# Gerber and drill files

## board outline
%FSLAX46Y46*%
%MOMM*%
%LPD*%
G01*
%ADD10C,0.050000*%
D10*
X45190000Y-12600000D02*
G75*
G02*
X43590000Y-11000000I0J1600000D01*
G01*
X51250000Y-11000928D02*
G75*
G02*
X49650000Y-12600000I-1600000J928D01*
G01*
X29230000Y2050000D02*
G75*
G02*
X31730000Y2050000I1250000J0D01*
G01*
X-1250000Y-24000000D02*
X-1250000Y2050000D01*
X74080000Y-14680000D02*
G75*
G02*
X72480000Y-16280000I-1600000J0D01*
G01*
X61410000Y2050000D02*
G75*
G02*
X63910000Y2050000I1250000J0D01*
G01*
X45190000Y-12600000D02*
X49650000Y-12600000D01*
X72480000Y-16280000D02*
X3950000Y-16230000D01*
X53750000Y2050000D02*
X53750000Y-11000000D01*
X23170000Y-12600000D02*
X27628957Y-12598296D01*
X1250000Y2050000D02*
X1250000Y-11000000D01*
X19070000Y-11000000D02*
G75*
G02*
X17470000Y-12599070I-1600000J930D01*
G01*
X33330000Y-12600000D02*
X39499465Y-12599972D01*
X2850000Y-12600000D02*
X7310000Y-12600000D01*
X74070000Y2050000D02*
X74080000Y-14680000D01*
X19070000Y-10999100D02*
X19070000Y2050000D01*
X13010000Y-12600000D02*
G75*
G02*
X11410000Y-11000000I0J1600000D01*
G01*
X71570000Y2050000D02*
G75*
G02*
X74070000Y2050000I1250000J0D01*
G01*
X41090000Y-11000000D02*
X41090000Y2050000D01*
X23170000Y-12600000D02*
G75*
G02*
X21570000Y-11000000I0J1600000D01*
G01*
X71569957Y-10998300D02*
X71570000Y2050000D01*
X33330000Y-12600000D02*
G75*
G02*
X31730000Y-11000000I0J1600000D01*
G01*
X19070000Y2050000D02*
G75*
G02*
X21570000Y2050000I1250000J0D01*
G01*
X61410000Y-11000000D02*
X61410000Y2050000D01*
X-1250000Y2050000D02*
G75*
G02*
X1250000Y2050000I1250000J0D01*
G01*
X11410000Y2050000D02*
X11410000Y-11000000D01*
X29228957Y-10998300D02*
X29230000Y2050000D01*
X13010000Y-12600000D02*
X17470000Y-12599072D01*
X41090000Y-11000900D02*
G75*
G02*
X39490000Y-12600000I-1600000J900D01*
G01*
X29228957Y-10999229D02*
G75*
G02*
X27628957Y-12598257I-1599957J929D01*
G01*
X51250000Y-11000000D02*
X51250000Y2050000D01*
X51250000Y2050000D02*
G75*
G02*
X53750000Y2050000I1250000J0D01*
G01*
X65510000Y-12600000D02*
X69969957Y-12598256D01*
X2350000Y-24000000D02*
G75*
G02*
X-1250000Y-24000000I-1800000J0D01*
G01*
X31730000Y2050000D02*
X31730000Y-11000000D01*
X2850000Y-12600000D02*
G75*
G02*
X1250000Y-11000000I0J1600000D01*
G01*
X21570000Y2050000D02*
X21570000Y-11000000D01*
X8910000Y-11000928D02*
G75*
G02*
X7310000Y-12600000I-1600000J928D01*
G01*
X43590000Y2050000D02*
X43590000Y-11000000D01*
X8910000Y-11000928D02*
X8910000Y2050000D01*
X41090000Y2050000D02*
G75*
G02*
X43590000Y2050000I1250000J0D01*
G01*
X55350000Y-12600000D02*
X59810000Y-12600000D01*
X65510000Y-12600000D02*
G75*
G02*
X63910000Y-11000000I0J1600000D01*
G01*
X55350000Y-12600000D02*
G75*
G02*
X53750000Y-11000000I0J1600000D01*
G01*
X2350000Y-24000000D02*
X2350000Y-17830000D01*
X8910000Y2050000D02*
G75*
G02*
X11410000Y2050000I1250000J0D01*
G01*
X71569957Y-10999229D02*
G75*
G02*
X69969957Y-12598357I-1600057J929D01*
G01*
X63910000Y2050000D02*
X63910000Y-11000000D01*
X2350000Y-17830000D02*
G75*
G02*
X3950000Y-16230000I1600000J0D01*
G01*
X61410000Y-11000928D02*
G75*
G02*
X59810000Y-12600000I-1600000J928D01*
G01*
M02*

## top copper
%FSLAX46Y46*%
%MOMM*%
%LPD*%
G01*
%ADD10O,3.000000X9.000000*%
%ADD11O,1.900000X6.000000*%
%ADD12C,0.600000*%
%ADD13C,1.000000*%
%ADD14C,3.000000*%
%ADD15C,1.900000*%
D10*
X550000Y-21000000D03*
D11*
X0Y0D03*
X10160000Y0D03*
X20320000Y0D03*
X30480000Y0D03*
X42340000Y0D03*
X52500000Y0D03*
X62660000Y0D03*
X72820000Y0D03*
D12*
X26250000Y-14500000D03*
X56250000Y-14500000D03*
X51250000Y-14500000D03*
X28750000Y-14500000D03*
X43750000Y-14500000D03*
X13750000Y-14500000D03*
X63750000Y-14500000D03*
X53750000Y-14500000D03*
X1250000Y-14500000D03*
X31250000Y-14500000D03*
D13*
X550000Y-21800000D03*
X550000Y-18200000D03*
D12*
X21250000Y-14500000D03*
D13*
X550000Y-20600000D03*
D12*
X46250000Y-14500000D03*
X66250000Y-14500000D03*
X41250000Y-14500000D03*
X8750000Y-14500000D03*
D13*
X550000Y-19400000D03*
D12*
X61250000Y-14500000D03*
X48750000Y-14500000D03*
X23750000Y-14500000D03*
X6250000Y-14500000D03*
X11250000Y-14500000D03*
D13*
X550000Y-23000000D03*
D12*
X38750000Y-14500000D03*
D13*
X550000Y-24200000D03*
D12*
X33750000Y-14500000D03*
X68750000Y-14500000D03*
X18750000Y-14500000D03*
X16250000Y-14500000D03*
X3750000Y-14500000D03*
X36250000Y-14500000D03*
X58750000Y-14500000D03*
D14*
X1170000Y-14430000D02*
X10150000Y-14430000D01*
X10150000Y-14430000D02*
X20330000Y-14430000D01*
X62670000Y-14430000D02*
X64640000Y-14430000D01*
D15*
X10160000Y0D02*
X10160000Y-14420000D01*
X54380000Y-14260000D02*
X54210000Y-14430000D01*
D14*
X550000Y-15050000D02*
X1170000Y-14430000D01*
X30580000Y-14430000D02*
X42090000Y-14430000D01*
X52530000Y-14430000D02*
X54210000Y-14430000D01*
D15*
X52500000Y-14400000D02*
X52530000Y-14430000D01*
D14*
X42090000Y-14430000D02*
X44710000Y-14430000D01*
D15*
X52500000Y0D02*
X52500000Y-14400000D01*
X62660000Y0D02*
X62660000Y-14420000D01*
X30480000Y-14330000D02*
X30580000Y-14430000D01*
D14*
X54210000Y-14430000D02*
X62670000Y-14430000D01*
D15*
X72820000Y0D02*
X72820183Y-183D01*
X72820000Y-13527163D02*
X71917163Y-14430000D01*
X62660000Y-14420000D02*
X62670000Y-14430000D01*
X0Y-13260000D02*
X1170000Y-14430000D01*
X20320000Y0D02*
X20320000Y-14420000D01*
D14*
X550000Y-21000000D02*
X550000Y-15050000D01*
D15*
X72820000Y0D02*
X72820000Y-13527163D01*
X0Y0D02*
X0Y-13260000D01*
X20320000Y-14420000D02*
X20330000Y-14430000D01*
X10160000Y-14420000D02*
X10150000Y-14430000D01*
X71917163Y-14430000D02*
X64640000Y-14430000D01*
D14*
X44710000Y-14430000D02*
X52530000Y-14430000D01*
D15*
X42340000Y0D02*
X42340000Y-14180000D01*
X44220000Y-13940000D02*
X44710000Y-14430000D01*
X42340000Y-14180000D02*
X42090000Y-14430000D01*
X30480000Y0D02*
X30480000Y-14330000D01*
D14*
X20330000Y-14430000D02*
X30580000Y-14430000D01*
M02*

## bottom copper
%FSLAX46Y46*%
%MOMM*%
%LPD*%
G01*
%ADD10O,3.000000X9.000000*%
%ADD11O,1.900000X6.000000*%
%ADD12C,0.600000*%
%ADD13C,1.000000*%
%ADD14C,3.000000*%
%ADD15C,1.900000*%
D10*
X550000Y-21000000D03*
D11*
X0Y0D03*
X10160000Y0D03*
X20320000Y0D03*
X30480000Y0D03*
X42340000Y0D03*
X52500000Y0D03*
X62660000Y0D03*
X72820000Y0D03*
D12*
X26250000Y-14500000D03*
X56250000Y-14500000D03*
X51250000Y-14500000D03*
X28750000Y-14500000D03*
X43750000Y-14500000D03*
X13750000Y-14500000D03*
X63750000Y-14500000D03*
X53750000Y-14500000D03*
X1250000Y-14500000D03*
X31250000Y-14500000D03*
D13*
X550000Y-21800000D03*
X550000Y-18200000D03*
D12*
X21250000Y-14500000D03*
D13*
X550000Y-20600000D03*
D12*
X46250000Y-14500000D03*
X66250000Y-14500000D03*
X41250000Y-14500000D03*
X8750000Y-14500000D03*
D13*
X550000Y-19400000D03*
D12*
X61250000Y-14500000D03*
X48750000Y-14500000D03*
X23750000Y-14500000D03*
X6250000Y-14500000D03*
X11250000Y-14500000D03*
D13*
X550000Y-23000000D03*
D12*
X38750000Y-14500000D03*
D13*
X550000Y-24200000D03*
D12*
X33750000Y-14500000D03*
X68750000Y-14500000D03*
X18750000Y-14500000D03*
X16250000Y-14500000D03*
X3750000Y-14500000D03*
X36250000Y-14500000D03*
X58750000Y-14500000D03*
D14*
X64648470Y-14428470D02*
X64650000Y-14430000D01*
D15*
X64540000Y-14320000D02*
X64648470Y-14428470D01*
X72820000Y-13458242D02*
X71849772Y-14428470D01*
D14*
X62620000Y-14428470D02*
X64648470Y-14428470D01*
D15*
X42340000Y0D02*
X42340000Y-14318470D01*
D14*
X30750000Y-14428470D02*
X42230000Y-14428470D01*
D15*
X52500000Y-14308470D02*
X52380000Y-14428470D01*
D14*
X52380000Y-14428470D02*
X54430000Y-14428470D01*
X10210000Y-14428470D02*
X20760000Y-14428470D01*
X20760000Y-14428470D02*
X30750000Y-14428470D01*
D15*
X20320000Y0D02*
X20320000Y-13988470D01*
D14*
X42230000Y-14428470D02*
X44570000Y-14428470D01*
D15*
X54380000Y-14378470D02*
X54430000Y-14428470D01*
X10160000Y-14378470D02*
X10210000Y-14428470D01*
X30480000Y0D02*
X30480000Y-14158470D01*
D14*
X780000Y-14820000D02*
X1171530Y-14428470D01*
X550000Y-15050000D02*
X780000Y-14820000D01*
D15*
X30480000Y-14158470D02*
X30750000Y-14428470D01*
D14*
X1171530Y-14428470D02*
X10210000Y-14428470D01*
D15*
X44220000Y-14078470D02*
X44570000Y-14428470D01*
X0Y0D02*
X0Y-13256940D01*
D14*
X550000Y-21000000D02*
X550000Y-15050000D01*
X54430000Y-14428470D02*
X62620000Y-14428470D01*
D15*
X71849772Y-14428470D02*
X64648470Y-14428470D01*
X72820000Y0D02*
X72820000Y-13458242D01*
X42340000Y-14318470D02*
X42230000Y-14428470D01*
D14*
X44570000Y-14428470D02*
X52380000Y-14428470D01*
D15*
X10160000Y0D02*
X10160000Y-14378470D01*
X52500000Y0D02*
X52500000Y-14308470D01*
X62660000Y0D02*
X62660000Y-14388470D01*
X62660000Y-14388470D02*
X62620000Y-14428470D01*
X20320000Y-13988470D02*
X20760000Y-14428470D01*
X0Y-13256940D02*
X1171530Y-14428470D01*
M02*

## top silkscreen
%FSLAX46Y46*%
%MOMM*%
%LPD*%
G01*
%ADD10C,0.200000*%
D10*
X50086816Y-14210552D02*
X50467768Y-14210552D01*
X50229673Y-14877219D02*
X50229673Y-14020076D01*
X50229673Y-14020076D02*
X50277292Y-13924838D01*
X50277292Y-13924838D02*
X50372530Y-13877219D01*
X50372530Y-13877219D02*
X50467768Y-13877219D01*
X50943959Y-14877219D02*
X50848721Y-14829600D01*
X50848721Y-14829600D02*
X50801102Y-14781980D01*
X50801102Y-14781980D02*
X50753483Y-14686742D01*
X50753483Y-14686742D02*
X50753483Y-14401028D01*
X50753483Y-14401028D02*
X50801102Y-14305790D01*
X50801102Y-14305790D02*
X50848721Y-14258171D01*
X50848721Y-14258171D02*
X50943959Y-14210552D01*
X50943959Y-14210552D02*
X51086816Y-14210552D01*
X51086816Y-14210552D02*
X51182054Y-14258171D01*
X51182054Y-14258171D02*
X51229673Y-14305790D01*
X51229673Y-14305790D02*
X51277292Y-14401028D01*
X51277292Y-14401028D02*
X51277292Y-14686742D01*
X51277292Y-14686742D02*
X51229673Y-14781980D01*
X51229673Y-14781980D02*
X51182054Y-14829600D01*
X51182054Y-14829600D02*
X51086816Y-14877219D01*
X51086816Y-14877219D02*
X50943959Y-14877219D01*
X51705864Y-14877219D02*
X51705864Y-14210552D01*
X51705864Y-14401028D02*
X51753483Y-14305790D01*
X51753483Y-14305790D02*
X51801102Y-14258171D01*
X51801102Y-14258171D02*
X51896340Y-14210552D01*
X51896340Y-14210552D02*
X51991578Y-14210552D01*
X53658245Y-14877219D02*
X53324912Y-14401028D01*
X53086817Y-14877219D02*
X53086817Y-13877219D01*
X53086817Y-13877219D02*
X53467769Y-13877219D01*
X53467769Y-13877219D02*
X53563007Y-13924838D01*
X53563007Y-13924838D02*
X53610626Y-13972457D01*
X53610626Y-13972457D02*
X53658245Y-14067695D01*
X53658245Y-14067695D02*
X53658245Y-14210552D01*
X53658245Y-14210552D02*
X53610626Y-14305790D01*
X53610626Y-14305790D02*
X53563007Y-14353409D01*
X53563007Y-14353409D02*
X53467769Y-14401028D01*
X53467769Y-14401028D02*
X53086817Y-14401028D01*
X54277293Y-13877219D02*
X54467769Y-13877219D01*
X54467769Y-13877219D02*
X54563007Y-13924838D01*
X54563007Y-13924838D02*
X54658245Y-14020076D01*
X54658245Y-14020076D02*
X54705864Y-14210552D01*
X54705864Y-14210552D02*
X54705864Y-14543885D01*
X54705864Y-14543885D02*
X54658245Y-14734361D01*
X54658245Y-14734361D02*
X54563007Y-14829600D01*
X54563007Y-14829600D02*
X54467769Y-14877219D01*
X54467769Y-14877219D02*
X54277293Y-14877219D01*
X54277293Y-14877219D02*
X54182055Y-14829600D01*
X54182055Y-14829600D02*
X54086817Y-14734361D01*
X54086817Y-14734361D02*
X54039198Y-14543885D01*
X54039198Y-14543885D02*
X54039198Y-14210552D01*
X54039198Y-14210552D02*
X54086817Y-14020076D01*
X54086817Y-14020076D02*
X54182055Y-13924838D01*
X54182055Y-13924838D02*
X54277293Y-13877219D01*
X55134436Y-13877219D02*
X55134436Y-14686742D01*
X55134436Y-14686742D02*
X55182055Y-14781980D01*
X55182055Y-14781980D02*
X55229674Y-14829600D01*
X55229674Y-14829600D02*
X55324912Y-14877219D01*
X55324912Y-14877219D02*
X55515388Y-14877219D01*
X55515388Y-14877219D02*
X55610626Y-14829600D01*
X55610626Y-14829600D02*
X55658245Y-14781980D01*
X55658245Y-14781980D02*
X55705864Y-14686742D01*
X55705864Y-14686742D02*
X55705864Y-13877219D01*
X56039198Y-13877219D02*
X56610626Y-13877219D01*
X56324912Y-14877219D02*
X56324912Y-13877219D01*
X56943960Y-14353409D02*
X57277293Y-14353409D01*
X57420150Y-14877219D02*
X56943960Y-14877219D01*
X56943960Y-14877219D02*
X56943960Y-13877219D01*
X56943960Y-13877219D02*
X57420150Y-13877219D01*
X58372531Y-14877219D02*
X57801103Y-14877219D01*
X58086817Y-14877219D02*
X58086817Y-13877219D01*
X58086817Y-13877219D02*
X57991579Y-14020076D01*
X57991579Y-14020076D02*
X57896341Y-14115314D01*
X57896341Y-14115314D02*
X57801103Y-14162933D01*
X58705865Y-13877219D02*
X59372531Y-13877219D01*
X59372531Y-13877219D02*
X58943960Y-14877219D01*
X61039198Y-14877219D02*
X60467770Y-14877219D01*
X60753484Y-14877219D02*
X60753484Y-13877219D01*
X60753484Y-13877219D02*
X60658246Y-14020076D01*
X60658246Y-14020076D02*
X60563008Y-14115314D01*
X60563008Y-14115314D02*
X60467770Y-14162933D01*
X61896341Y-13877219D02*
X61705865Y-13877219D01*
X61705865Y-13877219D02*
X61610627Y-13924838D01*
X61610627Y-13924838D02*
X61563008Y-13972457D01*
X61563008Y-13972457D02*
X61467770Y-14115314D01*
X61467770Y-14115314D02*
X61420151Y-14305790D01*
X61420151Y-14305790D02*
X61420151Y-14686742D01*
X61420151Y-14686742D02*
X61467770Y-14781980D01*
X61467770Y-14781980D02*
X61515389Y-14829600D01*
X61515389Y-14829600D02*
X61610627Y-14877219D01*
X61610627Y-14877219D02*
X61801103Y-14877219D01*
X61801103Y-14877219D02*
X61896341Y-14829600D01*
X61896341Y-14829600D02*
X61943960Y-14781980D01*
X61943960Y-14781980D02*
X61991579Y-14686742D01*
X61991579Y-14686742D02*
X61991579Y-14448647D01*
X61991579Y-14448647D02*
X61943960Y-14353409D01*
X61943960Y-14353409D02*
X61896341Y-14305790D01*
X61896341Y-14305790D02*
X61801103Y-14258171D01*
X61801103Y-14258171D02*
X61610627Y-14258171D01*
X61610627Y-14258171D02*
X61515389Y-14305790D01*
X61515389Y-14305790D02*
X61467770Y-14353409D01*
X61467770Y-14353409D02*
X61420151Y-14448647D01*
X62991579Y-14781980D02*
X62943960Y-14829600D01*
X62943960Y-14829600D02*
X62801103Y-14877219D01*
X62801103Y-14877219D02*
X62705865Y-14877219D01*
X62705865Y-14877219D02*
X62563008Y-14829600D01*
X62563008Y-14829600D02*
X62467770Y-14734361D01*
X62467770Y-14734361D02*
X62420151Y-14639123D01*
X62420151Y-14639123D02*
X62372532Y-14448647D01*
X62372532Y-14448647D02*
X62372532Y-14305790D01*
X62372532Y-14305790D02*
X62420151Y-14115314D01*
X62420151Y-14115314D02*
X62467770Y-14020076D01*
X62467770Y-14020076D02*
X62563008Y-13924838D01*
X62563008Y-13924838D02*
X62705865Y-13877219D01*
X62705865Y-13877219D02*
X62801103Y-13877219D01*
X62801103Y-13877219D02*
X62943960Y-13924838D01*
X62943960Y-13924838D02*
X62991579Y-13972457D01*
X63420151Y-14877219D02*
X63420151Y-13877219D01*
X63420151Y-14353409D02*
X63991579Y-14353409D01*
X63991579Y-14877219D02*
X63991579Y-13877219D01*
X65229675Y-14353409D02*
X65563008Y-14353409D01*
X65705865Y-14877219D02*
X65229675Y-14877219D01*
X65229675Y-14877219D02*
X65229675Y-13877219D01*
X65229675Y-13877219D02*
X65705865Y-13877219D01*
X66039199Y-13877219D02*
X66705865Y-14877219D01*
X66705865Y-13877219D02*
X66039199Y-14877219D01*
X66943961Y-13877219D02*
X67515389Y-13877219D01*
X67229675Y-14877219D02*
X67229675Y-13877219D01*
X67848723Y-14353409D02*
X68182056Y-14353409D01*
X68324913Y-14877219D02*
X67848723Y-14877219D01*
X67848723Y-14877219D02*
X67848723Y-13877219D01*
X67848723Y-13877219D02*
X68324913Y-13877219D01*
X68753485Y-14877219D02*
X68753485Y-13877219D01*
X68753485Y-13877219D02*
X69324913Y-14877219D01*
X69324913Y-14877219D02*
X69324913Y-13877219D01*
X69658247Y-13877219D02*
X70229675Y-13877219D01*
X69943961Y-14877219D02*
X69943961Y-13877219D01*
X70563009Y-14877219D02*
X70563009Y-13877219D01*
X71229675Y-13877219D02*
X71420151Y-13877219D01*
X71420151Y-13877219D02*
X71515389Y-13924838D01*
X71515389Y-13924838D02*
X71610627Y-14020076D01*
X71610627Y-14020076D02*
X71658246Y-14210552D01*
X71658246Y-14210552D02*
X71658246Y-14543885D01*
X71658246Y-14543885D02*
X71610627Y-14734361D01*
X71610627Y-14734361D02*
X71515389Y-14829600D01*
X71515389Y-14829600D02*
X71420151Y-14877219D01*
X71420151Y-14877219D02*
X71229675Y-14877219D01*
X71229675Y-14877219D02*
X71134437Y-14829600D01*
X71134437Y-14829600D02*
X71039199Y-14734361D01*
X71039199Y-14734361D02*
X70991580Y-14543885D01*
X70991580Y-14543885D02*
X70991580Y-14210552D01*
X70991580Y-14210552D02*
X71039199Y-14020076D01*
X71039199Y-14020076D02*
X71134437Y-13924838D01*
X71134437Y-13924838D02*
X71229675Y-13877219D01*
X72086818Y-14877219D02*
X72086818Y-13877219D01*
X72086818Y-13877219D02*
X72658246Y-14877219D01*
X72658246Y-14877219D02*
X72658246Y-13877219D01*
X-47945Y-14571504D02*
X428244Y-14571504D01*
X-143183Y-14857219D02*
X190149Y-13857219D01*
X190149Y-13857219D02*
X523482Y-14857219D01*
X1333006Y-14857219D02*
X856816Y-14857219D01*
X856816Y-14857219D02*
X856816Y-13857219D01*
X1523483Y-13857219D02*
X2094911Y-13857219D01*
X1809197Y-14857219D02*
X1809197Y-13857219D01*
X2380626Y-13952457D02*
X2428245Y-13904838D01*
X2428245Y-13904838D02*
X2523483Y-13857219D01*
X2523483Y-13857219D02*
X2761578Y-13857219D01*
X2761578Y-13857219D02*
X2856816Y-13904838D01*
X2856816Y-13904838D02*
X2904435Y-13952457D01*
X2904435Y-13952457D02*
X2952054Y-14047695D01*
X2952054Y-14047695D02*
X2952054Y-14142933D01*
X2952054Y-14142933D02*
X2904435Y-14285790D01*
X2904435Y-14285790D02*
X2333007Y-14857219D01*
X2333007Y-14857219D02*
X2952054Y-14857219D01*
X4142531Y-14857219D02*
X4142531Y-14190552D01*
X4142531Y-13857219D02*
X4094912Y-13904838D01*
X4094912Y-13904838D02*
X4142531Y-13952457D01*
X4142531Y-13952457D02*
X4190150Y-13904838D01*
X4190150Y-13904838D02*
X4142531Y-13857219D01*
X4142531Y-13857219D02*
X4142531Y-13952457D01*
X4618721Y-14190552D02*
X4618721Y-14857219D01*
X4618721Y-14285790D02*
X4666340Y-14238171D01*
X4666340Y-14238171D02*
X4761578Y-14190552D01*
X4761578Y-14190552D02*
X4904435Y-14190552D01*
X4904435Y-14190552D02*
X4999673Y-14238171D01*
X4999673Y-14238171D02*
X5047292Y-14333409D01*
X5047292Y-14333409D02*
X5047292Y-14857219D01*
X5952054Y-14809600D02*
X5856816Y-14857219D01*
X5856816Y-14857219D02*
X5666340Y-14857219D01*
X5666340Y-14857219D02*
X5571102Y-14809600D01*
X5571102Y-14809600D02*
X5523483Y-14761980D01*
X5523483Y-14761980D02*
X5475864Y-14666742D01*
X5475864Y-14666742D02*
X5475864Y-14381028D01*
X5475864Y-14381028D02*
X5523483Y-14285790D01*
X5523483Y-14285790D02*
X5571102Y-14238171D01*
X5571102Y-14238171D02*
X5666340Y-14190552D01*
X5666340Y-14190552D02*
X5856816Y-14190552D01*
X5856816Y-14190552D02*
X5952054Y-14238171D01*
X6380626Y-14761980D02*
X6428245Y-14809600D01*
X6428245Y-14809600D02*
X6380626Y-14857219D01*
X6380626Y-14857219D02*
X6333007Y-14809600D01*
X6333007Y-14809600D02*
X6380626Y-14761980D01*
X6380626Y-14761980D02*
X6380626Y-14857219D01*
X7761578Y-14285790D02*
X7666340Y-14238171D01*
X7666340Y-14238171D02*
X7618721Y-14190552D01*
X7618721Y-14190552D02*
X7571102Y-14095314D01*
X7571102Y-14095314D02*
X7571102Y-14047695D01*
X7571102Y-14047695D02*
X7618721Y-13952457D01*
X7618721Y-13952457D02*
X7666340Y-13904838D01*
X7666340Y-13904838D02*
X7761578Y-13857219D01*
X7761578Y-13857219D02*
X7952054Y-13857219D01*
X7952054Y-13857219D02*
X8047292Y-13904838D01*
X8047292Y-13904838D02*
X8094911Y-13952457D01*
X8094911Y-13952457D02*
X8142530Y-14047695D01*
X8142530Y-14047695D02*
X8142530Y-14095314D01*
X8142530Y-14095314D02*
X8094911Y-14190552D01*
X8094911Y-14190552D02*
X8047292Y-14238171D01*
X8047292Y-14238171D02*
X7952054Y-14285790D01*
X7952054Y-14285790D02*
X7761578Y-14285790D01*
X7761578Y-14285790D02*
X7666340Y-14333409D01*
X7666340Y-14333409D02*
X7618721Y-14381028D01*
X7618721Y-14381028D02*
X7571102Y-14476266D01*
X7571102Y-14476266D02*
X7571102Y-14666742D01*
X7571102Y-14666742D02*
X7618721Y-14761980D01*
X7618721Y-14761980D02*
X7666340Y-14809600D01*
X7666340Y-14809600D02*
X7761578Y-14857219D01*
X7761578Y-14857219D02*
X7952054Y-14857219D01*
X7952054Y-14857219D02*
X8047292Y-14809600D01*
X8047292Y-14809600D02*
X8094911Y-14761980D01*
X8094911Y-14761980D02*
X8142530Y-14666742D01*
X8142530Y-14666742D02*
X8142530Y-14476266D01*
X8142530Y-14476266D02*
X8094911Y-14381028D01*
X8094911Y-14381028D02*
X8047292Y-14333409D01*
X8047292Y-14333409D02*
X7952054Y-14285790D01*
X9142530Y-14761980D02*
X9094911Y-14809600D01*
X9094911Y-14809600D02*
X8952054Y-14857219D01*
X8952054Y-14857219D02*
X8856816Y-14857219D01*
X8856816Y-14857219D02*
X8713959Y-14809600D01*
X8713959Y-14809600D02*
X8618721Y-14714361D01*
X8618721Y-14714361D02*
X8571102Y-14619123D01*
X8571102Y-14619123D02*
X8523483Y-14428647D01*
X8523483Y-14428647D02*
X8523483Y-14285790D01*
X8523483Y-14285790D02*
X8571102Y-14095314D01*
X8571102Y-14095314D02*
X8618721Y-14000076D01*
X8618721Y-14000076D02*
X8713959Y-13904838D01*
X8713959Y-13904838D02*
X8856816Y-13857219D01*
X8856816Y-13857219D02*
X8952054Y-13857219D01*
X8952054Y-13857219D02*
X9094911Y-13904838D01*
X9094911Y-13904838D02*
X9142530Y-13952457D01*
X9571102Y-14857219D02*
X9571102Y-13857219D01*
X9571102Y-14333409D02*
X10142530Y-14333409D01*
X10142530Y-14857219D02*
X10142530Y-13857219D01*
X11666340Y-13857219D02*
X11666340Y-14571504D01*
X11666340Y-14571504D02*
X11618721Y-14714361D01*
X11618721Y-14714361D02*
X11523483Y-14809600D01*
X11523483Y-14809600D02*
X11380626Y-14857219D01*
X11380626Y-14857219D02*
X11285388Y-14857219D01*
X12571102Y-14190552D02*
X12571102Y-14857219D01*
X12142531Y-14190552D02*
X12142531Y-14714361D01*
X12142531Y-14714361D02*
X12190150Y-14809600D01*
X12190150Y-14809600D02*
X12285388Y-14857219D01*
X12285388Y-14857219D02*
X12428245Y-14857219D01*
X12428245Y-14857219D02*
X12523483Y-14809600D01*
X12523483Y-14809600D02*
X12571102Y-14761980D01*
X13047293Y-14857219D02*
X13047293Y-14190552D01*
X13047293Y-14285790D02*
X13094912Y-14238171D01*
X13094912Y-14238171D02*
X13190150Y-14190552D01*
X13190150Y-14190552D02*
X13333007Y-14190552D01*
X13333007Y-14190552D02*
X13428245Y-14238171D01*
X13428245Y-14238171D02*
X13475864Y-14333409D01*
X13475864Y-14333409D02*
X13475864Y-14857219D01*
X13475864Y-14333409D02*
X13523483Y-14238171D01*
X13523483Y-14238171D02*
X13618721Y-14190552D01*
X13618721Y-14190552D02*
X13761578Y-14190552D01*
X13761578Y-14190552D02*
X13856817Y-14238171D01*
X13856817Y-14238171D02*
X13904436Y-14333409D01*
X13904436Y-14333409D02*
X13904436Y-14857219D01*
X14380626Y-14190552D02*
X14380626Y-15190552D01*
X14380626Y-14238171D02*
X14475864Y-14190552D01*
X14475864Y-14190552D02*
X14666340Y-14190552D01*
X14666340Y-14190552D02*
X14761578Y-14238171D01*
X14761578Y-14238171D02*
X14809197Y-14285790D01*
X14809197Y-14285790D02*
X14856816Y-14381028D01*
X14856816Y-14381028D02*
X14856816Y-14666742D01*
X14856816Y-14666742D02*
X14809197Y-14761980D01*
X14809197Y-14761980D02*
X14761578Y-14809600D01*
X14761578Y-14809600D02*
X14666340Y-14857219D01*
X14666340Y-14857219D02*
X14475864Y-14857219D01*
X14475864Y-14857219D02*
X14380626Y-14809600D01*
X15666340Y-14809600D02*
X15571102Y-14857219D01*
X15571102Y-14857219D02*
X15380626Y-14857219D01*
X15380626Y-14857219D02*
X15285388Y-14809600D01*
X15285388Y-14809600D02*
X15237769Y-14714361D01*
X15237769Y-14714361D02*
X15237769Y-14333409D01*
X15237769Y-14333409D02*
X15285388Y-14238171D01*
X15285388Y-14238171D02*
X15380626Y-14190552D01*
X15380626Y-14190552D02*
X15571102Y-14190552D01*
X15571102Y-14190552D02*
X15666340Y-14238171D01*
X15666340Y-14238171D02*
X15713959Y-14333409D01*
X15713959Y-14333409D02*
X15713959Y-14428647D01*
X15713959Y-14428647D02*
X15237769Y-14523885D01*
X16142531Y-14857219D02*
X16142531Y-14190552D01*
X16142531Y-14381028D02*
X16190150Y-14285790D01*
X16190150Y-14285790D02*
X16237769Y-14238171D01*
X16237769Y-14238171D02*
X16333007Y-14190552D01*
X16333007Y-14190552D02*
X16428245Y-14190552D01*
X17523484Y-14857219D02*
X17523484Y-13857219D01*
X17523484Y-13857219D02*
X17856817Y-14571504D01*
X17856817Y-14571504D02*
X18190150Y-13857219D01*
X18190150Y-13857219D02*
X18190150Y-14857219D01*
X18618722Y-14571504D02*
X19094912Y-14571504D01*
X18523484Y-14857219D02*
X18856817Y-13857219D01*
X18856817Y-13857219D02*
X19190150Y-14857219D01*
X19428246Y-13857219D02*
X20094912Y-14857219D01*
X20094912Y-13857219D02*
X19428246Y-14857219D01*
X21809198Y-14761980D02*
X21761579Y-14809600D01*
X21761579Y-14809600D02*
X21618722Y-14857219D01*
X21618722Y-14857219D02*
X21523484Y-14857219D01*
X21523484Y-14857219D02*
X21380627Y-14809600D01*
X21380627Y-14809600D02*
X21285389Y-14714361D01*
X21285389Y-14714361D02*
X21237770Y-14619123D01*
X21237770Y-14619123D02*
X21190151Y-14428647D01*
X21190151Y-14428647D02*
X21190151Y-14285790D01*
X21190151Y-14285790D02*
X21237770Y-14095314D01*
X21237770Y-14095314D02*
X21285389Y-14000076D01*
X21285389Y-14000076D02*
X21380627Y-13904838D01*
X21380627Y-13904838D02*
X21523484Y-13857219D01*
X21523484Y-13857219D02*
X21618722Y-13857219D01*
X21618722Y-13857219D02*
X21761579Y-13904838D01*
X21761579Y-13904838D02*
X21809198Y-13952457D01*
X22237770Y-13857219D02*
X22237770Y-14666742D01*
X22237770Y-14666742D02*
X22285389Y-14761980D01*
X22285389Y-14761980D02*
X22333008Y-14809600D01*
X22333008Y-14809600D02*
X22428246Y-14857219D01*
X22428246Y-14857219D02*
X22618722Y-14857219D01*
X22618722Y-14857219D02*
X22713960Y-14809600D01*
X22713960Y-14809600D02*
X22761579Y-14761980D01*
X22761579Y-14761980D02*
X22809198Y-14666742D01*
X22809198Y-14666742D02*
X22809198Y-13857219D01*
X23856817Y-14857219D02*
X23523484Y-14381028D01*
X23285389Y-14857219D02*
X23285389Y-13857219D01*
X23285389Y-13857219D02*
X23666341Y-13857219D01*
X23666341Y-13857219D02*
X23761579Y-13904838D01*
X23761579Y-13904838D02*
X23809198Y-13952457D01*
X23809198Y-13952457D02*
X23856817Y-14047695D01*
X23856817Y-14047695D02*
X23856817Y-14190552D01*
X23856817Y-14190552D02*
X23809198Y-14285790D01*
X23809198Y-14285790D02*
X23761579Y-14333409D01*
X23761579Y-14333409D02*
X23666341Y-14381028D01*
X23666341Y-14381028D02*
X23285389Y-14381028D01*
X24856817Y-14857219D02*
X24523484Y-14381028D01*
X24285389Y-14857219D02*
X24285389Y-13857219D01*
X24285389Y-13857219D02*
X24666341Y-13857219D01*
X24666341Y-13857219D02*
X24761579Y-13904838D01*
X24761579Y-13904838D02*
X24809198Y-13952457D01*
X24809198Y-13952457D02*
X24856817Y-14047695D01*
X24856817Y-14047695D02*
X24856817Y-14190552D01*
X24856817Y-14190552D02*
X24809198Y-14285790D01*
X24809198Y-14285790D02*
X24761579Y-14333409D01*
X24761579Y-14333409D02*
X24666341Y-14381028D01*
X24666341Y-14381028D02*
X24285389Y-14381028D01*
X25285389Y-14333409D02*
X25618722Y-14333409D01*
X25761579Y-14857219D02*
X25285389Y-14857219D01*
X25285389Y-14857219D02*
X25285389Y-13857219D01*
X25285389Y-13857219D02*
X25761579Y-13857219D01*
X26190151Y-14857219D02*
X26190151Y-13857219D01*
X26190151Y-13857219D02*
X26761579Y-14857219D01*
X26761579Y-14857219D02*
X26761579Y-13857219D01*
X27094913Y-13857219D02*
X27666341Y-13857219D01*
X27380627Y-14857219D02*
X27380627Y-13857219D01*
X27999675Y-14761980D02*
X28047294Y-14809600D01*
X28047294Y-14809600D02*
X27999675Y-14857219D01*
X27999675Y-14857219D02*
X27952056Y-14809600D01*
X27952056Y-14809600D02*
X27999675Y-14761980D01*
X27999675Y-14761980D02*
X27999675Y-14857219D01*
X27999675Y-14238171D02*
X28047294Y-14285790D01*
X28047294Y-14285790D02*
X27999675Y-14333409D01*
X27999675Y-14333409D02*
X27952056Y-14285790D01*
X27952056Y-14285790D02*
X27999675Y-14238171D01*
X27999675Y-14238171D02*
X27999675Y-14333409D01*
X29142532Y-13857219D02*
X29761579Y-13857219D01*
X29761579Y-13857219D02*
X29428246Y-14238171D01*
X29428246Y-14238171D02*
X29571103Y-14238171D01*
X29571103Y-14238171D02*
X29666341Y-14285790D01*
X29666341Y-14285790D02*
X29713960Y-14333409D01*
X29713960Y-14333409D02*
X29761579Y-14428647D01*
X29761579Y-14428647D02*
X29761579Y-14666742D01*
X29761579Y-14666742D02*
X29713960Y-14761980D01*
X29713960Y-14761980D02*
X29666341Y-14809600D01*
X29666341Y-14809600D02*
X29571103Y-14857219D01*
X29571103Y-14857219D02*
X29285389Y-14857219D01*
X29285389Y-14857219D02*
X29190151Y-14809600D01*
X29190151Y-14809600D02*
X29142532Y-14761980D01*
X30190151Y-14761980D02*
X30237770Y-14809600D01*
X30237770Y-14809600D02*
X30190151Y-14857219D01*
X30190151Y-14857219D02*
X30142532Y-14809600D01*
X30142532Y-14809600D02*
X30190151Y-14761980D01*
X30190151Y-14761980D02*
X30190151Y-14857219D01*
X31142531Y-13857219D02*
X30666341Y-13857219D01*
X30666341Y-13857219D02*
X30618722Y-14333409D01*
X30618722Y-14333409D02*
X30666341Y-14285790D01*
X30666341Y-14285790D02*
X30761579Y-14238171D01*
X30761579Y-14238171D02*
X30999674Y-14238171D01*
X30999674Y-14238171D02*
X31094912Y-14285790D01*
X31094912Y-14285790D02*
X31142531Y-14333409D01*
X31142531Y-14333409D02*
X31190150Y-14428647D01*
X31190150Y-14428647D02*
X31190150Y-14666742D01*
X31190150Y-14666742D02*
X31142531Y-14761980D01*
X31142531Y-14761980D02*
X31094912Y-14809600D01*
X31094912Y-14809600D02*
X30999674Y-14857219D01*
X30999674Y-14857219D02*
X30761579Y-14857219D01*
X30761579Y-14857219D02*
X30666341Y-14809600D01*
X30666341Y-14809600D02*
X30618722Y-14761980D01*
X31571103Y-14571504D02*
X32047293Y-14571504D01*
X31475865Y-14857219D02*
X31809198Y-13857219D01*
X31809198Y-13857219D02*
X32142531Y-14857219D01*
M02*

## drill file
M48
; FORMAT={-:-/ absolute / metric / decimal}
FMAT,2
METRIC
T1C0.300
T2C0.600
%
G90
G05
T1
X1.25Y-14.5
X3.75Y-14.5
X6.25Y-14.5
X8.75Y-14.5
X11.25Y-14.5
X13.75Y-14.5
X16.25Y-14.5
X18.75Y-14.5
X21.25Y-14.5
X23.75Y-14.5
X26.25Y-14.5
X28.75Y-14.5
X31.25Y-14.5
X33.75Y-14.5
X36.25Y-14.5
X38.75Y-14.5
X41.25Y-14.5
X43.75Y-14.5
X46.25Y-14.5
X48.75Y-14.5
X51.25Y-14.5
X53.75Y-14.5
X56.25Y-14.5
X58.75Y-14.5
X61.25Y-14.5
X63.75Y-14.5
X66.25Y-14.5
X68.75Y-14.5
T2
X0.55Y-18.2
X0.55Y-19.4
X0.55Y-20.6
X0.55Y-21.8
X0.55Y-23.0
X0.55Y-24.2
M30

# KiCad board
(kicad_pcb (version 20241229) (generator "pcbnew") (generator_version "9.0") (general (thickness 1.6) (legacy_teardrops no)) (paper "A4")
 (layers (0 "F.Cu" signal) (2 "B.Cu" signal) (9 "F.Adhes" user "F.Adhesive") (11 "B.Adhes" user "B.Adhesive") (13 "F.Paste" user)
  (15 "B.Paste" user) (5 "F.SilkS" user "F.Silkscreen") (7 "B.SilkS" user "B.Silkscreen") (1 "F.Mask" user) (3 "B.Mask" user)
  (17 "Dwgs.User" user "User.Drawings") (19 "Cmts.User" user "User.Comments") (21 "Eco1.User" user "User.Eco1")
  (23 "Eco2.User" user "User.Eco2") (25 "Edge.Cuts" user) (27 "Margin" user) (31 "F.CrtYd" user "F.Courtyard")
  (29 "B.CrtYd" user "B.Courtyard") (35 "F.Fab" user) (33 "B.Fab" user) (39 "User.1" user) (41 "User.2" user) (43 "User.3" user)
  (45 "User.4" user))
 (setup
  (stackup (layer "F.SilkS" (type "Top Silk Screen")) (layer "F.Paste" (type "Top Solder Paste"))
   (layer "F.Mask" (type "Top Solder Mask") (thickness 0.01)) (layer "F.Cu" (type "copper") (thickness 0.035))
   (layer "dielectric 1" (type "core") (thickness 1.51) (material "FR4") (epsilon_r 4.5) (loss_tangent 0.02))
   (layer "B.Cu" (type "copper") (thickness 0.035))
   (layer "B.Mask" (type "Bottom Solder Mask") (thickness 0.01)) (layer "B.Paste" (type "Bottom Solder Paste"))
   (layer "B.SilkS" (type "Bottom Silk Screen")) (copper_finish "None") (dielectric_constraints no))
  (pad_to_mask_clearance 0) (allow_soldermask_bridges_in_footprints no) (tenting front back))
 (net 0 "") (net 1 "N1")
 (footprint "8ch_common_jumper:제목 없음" (layer "F.Cu") (at 0.55 21)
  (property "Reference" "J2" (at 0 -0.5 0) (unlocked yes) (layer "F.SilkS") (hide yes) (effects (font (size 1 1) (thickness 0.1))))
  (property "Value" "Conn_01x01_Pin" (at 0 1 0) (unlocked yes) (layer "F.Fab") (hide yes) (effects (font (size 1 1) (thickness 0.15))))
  (pad "1" smd oval (at 0 0 90) (size 9 3) (layers "F.Cu" "F.Mask" "F.Paste") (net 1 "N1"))
  (pad "1" smd oval (at 0 0 270) (size 9 3) (layers "B.Cu" "B.Mask" "B.Paste") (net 1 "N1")))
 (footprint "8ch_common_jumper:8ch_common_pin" (layer "F.Cu") (at 0 0)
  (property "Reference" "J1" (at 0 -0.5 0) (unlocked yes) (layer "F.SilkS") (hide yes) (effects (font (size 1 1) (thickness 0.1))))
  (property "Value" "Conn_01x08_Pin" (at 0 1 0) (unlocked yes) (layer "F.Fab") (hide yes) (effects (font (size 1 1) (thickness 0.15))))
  (pad "1" smd oval (at 0 0 90) (size 6 1.9) (layers "F.Cu" "F.Mask" "F.Paste") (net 1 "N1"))
  (pad "1" smd oval (at 0 0 270) (size 6 1.9) (layers "B.Cu" "B.Mask" "B.Paste") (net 1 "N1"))
  (pad "2" smd oval (at 10.16 0 90) (size 6 1.9) (layers "F.Cu" "F.Mask" "F.Paste") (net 1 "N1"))
  (pad "2" smd oval (at 10.16 0 270) (size 6 1.9) (layers "B.Cu" "B.Mask" "B.Paste") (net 1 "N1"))
  (pad "3" smd oval (at 20.32 0 90) (size 6 1.9) (layers "F.Cu" "F.Mask" "F.Paste") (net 1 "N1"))
  (pad "3" smd oval (at 20.32 0 270) (size 6 1.9) (layers "B.Cu" "B.Mask" "B.Paste") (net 1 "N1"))
  (pad "4" smd oval (at 30.48 0 90) (size 6 1.9) (layers "F.Cu" "F.Mask" "F.Paste") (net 1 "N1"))
  (pad "4" smd oval (at 30.48 0 270) (size 6 1.9) (layers "B.Cu" "B.Mask" "B.Paste") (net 1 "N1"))
  (pad "5" smd oval (at 42.34 0 90) (size 6 1.9) (layers "F.Cu" "F.Mask" "F.Paste") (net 1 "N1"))
  (pad "5" smd oval (at 42.34 0 270) (size 6 1.9) (layers "B.Cu" "B.Mask" "B.Paste") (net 1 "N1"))
  (pad "6" smd oval (at 52.5 0 90) (size 6 1.9) (layers "F.Cu" "F.Mask" "F.Paste") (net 1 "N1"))
  (pad "6" smd oval (at 52.5 0 270) (size 6 1.9) (layers "B.Cu" "B.Mask" "B.Paste") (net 1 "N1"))
  (pad "7" smd oval (at 62.66 0 90) (size 6 1.9) (layers "F.Cu" "F.Mask" "F.Paste") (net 1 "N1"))
  (pad "7" smd oval (at 62.66 0 270) (size 6 1.9) (layers "B.Cu" "B.Mask" "B.Paste") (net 1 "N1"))
  (pad "8" smd oval (at 72.82 0 90) (size 6 1.9) (layers "F.Cu" "F.Mask" "F.Paste") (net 1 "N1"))
  (pad "8" smd oval (at 72.82 0 270) (size 6 1.9) (layers "B.Cu" "B.Mask" "B.Paste") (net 1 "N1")))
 (gr_arc (start 45.19 12.6) (mid 44.058629 12.131371) (end 43.59 11) (stroke (width 0.05) (type default)) (layer "Edge.Cuts"))
 (gr_arc (start 51.25 11.000928) (mid 50.781043 12.131699) (end 49.65 12.6) (stroke (width 0.05) (type default)) (layer "Edge.Cuts"))
 (gr_arc (start 29.23 -2.05) (mid 30.48 -3.3) (end 31.73 -2.05) (stroke (width 0.05) (type solid)) (layer "Edge.Cuts"))
 (gr_line (start -1.25 24) (end -1.25 -2.05) (stroke (width 0.05) (type default)) (layer "Edge.Cuts"))
 (gr_arc (start 74.08 14.68) (mid 73.611371 15.811371) (end 72.48 16.28) (stroke (width 0.05) (type solid)) (layer "Edge.Cuts"))
 (gr_arc (start 61.41 -2.05) (mid 62.66 -3.3) (end 63.91 -2.05) (stroke (width 0.05) (type solid)) (layer "Edge.Cuts"))
 (gr_line (start 45.19 12.6) (end 49.65 12.6) (stroke (width 0.05) (type default)) (layer "Edge.Cuts"))
 (gr_line (start 72.48 16.28) (end 3.95 16.23) (stroke (width 0.05) (type default)) (layer "Edge.Cuts"))
 (gr_line (start 53.75 -2.05) (end 53.75 11) (stroke (width 0.05) (type default)) (layer "Edge.Cuts"))
 (gr_line (start 23.17 12.6) (end 27.628957 12.598296) (stroke (width 0.05) (type default)) (layer "Edge.Cuts"))
 (gr_line (start 1.25 -2.05) (end 1.25 11) (stroke (width 0.05) (type default)) (layer "Edge.Cuts"))
 (gr_arc (start 19.07 11) (mid 18.601043 12.130771) (end 17.47 12.599072) (stroke (width 0.05) (type default)) (layer "Edge.Cuts"))
 (gr_line (start 33.33 12.6) (end 39.499465 12.599972) (stroke (width 0.05) (type default)) (layer "Edge.Cuts"))
 (gr_line (start 2.85 12.6) (end 7.31 12.6) (stroke (width 0.05) (type default)) (layer "Edge.Cuts"))
 (gr_line (start 74.07 -2.05) (end 74.08 14.68) (stroke (width 0.05) (type default)) (layer "Edge.Cuts"))
 (gr_line (start 19.07 10.9991) (end 19.07 -2.05) (stroke (width 0.05) (type default)) (layer "Edge.Cuts"))
 (gr_arc (start 13.01 12.6) (mid 11.878629 12.131371) (end 11.41 11) (stroke (width 0.05) (type default)) (layer "Edge.Cuts"))
 (gr_arc (start 71.57 -2.05) (mid 72.82 -3.3) (end 74.07 -2.05) (stroke (width 0.05) (type solid)) (layer "Edge.Cuts"))
 (gr_line (start 41.09 11) (end 41.09 -2.05) (stroke (width 0.05) (type default)) (layer "Edge.Cuts"))
 (gr_arc (start 23.17 12.6) (mid 22.038629 12.131371) (end 21.57 11) (stroke (width 0.05) (type default)) (layer "Edge.Cuts"))
 (gr_line (start 71.569957 10.9983) (end 71.57 -2.05) (stroke (width 0.05) (type default)) (layer "Edge.Cuts"))
 (gr_arc (start 33.33 12.6) (mid 32.198629 12.131371) (end 31.73 11) (stroke (width 0.05) (type default)) (layer "Edge.Cuts"))
 (gr_arc (start 19.07 -2.05) (mid 20.32 -3.3) (end 21.57 -2.05) (stroke (width 0.05) (type solid)) (layer "Edge.Cuts"))
 (gr_line (start 61.41 11) (end 61.41 -2.05) (stroke (width 0.05) (type default)) (layer "Edge.Cuts"))
 (gr_arc (start -1.25 -2.05) (mid 0 -3.3) (end 1.25 -2.05) (stroke (width 0.05) (type solid)) (layer "Edge.Cuts"))
 (gr_line (start 11.41 -2.05) (end 11.41 11) (stroke (width 0.05) (type default)) (layer "Edge.Cuts"))
 (gr_line (start 29.228957 10.9983) (end 29.23 -2.05) (stroke (width 0.05) (type default)) (layer "Edge.Cuts"))
 (gr_line (start 13.01 12.6) (end 17.47 12.599072) (stroke (width 0.05) (type default)) (layer "Edge.Cuts"))
 (gr_arc (start 41.09 11.0009) (mid 40.621053 12.131689) (end 39.49 12.599972) (stroke (width 0.05) (type default)) (layer "Edge.Cuts"))
 (gr_arc (start 29.228957 10.999229) (mid 28.76 12.13) (end 27.628957 12.598301) (stroke (width 0.05) (type default)) (layer "Edge.Cuts"))
 (gr_line (start 51.25 11) (end 51.25 -2.05) (stroke (width 0.05) (type default)) (layer "Edge.Cuts"))
 (gr_arc (start 51.25 -2.05) (mid 52.5 -3.3) (end 53.75 -2.05) (stroke (width 0.05) (type solid)) (layer "Edge.Cuts"))
 (gr_line (start 65.51 12.6) (end 69.969957 12.598256) (stroke (width 0.05) (type default)) (layer "Edge.Cuts"))
 (gr_arc (start 2.35 24) (mid 0.55 25.8) (end -1.25 24) (stroke (width 0.05) (type solid)) (layer "Edge.Cuts"))
 (gr_line (start 31.73 -2.05) (end 31.73 11) (stroke (width 0.05) (type default)) (layer "Edge.Cuts"))
 (gr_arc (start 2.85 12.6) (mid 1.718629 12.131371) (end 1.25 11) (stroke (width 0.05) (type default)) (layer "Edge.Cuts"))
 (gr_line (start 21.57 -2.05) (end 21.57 11) (stroke (width 0.05) (type default)) (layer "Edge.Cuts"))
 (gr_arc (start 8.91 11.000928) (mid 8.441043 12.131699) (end 7.31 12.6) (stroke (width 0.05) (type default)) (layer "Edge.Cuts"))
 (gr_line (start 43.59 -2.05) (end 43.59 11) (stroke (width 0.05) (type default)) (layer "Edge.Cuts"))
 (gr_line (start 8.91 11.000928) (end 8.91 -2.05) (stroke (width 0.05) (type default)) (layer "Edge.Cuts"))
 (gr_arc (start 41.09 -2.05) (mid 42.34 -3.3) (end 43.59 -2.05) (stroke (width 0.05) (type solid)) (layer "Edge.Cuts"))
 (gr_line (start 55.35 12.6) (end 59.81 12.6) (stroke (width 0.05) (type default)) (layer "Edge.Cuts"))
 (gr_arc (start 65.51 12.6) (mid 64.378629 12.131371) (end 63.91 11) (stroke (width 0.05) (type default)) (layer "Edge.Cuts"))
 (gr_arc (start 55.35 12.6) (mid 54.218629 12.131371) (end 53.75 11) (stroke (width 0.05) (type default)) (layer "Edge.Cuts"))
 (gr_line (start 2.35 24) (end 2.35 17.83) (stroke (width 0.05) (type default)) (layer "Edge.Cuts"))
 (gr_arc (start 8.91 -2.05) (mid 10.16 -3.3) (end 11.41 -2.05) (stroke (width 0.05) (type solid)) (layer "Edge.Cuts"))
 (gr_arc (start 71.569957 10.999229) (mid 71.100997 12.129984) (end 69.969957 12.598301) (stroke (width 0.05) (type default))
  (layer "Edge.Cuts"))
 (gr_line (start 63.91 -2.05) (end 63.91 11) (stroke (width 0.05) (type default)) (layer "Edge.Cuts"))
 (gr_arc (start 2.35 17.83) (mid 2.818629 16.698629) (end 3.95 16.23) (stroke (width 0.05) (type solid)) (layer "Edge.Cuts"))
 (gr_arc (start 61.41 11.000928) (mid 60.941043 12.131699) (end 59.81 12.6) (stroke (width 0.05) (type default)) (layer "Edge.Cuts"))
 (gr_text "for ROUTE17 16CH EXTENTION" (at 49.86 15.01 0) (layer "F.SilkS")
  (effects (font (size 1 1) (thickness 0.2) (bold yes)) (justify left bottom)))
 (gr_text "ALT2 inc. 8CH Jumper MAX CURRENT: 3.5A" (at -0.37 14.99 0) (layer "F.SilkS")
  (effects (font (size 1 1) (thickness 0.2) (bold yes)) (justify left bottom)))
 (segment (start 1.17 14.43) (end 10.15 14.43) (width 3) (layer "F.Cu") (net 1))
 (segment (start 10.15 14.43) (end 20.33 14.43) (width 3) (layer "F.Cu") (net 1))
 (segment (start 62.67 14.43) (end 64.64 14.43) (width 3) (layer "F.Cu") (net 1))
 (segment (start 10.16 0) (end 10.16 14.42) (width 1.9) (layer "F.Cu") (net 1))
 (segment (start 54.38 14.26) (end 54.21 14.43) (width 1.9) (layer "F.Cu") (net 1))
 (segment (start 0.55 15.05) (end 1.17 14.43) (width 3) (layer "F.Cu") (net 1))
 (segment (start 30.58 14.43) (end 42.09 14.43) (width 3) (layer "F.Cu") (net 1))
 (segment (start 52.53 14.43) (end 54.21 14.43) (width 3) (layer "F.Cu") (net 1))
 (segment (start 52.5 14.4) (end 52.53 14.43) (width 1.9) (layer "F.Cu") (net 1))
 (segment (start 42.09 14.43) (end 44.71 14.43) (width 3) (layer "F.Cu") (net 1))
 (segment (start 52.5 0) (end 52.5 14.4) (width 1.9) (layer "F.Cu") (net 1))
 (segment (start 62.66 0) (end 62.66 14.42) (width 1.9) (layer "F.Cu") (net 1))
 (segment (start 30.48 14.33) (end 30.58 14.43) (width 1.9) (layer "F.Cu") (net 1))
 (segment (start 54.21 14.43) (end 62.67 14.43) (width 3) (layer "F.Cu") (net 1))
 (segment (start 72.82 0) (end 72.820183 0.000183) (width 1.9) (layer "F.Cu") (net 1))
 (segment (start 72.82 13.527163) (end 71.917163 14.43) (width 1.9) (layer "F.Cu") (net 1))
 (segment (start 62.66 14.42) (end 62.67 14.43) (width 1.9) (layer "F.Cu") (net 1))
 (segment (start 0 13.26) (end 1.17 14.43) (width 1.9) (layer "F.Cu") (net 1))
 (segment (start 20.32 0) (end 20.32 14.42) (width 1.9) (layer "F.Cu") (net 1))
 (segment (start 0.55 21) (end 0.55 15.05) (width 3) (layer "F.Cu") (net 1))
 (segment (start 72.82 0) (end 72.82 13.527163) (width 1.9) (layer "F.Cu") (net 1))
 (segment (start 0 0) (end 0 13.26) (width 1.9) (layer "F.Cu") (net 1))
 (segment (start 20.32 14.42) (end 20.33 14.43) (width 1.9) (layer "F.Cu") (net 1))
 (segment (start 10.16 14.42) (end 10.15 14.43) (width 1.9) (layer "F.Cu") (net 1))
 (segment (start 71.917163 14.43) (end 64.64 14.43) (width 1.9) (layer "F.Cu") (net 1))
 (segment (start 44.71 14.43) (end 52.53 14.43) (width 3) (layer "F.Cu") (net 1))
 (segment (start 42.34 0) (end 42.34 14.18) (width 1.9) (layer "F.Cu") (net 1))
 (segment (start 44.22 13.94) (end 44.71 14.43) (width 1.9) (layer "F.Cu") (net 1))
 (segment (start 42.34 14.18) (end 42.09 14.43) (width 1.9) (layer "F.Cu") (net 1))
 (segment (start 30.48 0) (end 30.48 14.33) (width 1.9) (layer "F.Cu") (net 1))
 (segment (start 20.33 14.43) (end 30.58 14.43) (width 3) (layer "F.Cu") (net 1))
 (via (at 26.25 14.5) (size 0.6) (drill 0.3) (layers "F.Cu" "B.Cu") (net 1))
 (via (at 56.25 14.5) (size 0.6) (drill 0.3) (layers "F.Cu" "B.Cu") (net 1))
 (via (at 51.25 14.5) (size 0.6) (drill 0.3) (layers "F.Cu" "B.Cu") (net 1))
 (via (at 28.75 14.5) (size 0.6) (drill 0.3) (layers "F.Cu" "B.Cu") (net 1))
 (via (at 43.75 14.5) (size 0.6) (drill 0.3) (layers "F.Cu" "B.Cu") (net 1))
 (via (at 13.75 14.5) (size 0.6) (drill 0.3) (layers "F.Cu" "B.Cu") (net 1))
 (via (at 63.75 14.5) (size 0.6) (drill 0.3) (layers "F.Cu" "B.Cu") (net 1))
 (via (at 53.75 14.5) (size 0.6) (drill 0.3) (layers "F.Cu" "B.Cu") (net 1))
 (via (at 1.25 14.5) (size 0.6) (drill 0.3) (layers "F.Cu" "B.Cu") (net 1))
 (via (at 31.25 14.5) (size 0.6) (drill 0.3) (layers "F.Cu" "B.Cu") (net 1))
 (via (at 0.55 21.8) (size 1) (drill 0.6) (layers "F.Cu" "B.Cu") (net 1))
 (via (at 0.55 18.2) (size 1) (drill 0.6) (layers "F.Cu" "B.Cu") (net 1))
 (via (at 21.25 14.5) (size 0.6) (drill 0.3) (layers "F.Cu" "B.Cu") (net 1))
 (via (at 0.55 20.6) (size 1) (drill 0.6) (layers "F.Cu" "B.Cu") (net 1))
 (via (at 46.25 14.5) (size 0.6) (drill 0.3) (layers "F.Cu" "B.Cu") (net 1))
 (via (at 66.25 14.5) (size 0.6) (drill 0.3) (layers "F.Cu" "B.Cu") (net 1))
 (via (at 41.25 14.5) (size 0.6) (drill 0.3) (layers "F.Cu" "B.Cu") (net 1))
 (via (at 8.75 14.5) (size 0.6) (drill 0.3) (layers "F.Cu" "B.Cu") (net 1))
 (via (at 0.55 19.4) (size 1) (drill 0.6) (layers "F.Cu" "B.Cu") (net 1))
 (via (at 61.25 14.5) (size 0.6) (drill 0.3) (layers "F.Cu" "B.Cu") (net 1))
 (via (at 48.75 14.5) (size 0.6) (drill 0.3) (layers "F.Cu" "B.Cu") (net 1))
 (via (at 23.75 14.5) (size 0.6) (drill 0.3) (layers "F.Cu" "B.Cu") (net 1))
 (via (at 6.25 14.5) (size 0.6) (drill 0.3) (layers "F.Cu" "B.Cu") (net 1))
 (via (at 11.25 14.5) (size 0.6) (drill 0.3) (layers "F.Cu" "B.Cu") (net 1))
 (via (at 0.55 23) (size 1) (drill 0.6) (layers "F.Cu" "B.Cu") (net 1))
 (via (at 38.75 14.5) (size 0.6) (drill 0.3) (layers "F.Cu" "B.Cu") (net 1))
 (via (at 0.55 24.2) (size 1) (drill 0.6) (layers "F.Cu" "B.Cu") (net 1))
 (via (at 33.75 14.5) (size 0.6) (drill 0.3) (layers "F.Cu" "B.Cu") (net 1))
 (via (at 68.75 14.5) (size 0.6) (drill 0.3) (layers "F.Cu" "B.Cu") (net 1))
 (via (at 18.75 14.5) (size 0.6) (drill 0.3) (layers "F.Cu" "B.Cu") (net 1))
 (via (at 16.25 14.5) (size 0.6) (drill 0.3) (layers "F.Cu" "B.Cu") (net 1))
 (via (at 3.75 14.5) (size 0.6) (drill 0.3) (layers "F.Cu" "B.Cu") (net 1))
 (via (at 36.25 14.5) (size 0.6) (drill 0.3) (layers "F.Cu" "B.Cu") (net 1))
 (via (at 58.75 14.5) (size 0.6) (drill 0.3) (layers "F.Cu" "B.Cu") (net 1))
 (segment (start 64.64847 14.42847) (end 64.65 14.43) (width 3) (layer "B.Cu") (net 1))
 (segment (start 64.54 14.32) (end 64.64847 14.42847) (width 1.9) (layer "B.Cu") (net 1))
 (segment (start 72.82 13.458242) (end 71.849772 14.42847) (width 1.9) (layer "B.Cu") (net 1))
 (segment (start 62.62 14.42847) (end 64.64847 14.42847) (width 3) (layer "B.Cu") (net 1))
 (segment (start 42.34 0) (end 42.34 14.31847) (width 1.9) (layer "B.Cu") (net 1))
 (segment (start 30.75 14.42847) (end 42.23 14.42847) (width 3) (layer "B.Cu") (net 1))
 (segment (start 52.5 14.30847) (end 52.38 14.42847) (width 1.9) (layer "B.Cu") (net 1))
 (segment (start 52.38 14.42847) (end 54.43 14.42847) (width 3) (layer "B.Cu") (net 1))
 (segment (start 10.21 14.42847) (end 20.76 14.42847) (width 3) (layer "B.Cu") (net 1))
 (segment (start 20.76 14.42847) (end 30.75 14.42847) (width 3) (layer "B.Cu") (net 1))
 (segment (start 20.32 0) (end 20.32 13.98847) (width 1.9) (layer "B.Cu") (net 1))
 (segment (start 42.23 14.42847) (end 44.57 14.42847) (width 3) (layer "B.Cu") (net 1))
 (segment (start 54.38 14.37847) (end 54.43 14.42847) (width 1.9) (layer "B.Cu") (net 1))
 (segment (start 10.16 14.37847) (end 10.21 14.42847) (width 1.9) (layer "B.Cu") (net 1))
 (segment (start 30.48 0) (end 30.48 14.15847) (width 1.9) (layer "B.Cu") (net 1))
 (segment (start 0.78 14.82) (end 1.17153 14.42847) (width 3) (layer "B.Cu") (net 1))
 (segment (start 0.55 15.05) (end 0.78 14.82) (width 3) (layer "B.Cu") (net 1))
 (segment (start 30.48 14.15847) (end 30.75 14.42847) (width 1.9) (layer "B.Cu") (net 1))
 (segment (start 1.17153 14.42847) (end 10.21 14.42847) (width 3) (layer "B.Cu") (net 1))
 (segment (start 44.22 14.07847) (end 44.57 14.42847) (width 1.9) (layer "B.Cu") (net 1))
 (segment (start 0 0) (end 0 13.25694) (width 1.9) (layer "B.Cu") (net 1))
 (segment (start 0.55 21) (end 0.55 15.05) (width 3) (layer "B.Cu") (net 1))
 (segment (start 54.43 14.42847) (end 62.62 14.42847) (width 3) (layer "B.Cu") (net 1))
 (segment (start 71.849772 14.42847) (end 64.64847 14.42847) (width 1.9) (layer "B.Cu") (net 1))
 (segment (start 72.82 0) (end 72.82 13.458242) (width 1.9) (layer "B.Cu") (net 1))
 (segment (start 42.34 14.31847) (end 42.23 14.42847) (width 1.9) (layer "B.Cu") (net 1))
 (segment (start 44.57 14.42847) (end 52.38 14.42847) (width 3) (layer "B.Cu") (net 1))
 (segment (start 10.16 0) (end 10.16 14.37847) (width 1.9) (layer "B.Cu") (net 1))
 (segment (start 52.5 0) (end 52.5 14.30847) (width 1.9) (layer "B.Cu") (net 1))
 (segment (start 62.66 0) (end 62.66 14.38847) (width 1.9) (layer "B.Cu") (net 1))
 (segment (start 62.66 14.38847) (end 62.62 14.42847) (width 1.9) (layer "B.Cu") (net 1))
 (segment (start 20.32 13.98847) (end 20.76 14.42847) (width 1.9) (layer "B.Cu") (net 1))
 (segment (start 0 13.25694) (end 1.17153 14.42847) (width 1.9) (layer "B.Cu") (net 1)))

